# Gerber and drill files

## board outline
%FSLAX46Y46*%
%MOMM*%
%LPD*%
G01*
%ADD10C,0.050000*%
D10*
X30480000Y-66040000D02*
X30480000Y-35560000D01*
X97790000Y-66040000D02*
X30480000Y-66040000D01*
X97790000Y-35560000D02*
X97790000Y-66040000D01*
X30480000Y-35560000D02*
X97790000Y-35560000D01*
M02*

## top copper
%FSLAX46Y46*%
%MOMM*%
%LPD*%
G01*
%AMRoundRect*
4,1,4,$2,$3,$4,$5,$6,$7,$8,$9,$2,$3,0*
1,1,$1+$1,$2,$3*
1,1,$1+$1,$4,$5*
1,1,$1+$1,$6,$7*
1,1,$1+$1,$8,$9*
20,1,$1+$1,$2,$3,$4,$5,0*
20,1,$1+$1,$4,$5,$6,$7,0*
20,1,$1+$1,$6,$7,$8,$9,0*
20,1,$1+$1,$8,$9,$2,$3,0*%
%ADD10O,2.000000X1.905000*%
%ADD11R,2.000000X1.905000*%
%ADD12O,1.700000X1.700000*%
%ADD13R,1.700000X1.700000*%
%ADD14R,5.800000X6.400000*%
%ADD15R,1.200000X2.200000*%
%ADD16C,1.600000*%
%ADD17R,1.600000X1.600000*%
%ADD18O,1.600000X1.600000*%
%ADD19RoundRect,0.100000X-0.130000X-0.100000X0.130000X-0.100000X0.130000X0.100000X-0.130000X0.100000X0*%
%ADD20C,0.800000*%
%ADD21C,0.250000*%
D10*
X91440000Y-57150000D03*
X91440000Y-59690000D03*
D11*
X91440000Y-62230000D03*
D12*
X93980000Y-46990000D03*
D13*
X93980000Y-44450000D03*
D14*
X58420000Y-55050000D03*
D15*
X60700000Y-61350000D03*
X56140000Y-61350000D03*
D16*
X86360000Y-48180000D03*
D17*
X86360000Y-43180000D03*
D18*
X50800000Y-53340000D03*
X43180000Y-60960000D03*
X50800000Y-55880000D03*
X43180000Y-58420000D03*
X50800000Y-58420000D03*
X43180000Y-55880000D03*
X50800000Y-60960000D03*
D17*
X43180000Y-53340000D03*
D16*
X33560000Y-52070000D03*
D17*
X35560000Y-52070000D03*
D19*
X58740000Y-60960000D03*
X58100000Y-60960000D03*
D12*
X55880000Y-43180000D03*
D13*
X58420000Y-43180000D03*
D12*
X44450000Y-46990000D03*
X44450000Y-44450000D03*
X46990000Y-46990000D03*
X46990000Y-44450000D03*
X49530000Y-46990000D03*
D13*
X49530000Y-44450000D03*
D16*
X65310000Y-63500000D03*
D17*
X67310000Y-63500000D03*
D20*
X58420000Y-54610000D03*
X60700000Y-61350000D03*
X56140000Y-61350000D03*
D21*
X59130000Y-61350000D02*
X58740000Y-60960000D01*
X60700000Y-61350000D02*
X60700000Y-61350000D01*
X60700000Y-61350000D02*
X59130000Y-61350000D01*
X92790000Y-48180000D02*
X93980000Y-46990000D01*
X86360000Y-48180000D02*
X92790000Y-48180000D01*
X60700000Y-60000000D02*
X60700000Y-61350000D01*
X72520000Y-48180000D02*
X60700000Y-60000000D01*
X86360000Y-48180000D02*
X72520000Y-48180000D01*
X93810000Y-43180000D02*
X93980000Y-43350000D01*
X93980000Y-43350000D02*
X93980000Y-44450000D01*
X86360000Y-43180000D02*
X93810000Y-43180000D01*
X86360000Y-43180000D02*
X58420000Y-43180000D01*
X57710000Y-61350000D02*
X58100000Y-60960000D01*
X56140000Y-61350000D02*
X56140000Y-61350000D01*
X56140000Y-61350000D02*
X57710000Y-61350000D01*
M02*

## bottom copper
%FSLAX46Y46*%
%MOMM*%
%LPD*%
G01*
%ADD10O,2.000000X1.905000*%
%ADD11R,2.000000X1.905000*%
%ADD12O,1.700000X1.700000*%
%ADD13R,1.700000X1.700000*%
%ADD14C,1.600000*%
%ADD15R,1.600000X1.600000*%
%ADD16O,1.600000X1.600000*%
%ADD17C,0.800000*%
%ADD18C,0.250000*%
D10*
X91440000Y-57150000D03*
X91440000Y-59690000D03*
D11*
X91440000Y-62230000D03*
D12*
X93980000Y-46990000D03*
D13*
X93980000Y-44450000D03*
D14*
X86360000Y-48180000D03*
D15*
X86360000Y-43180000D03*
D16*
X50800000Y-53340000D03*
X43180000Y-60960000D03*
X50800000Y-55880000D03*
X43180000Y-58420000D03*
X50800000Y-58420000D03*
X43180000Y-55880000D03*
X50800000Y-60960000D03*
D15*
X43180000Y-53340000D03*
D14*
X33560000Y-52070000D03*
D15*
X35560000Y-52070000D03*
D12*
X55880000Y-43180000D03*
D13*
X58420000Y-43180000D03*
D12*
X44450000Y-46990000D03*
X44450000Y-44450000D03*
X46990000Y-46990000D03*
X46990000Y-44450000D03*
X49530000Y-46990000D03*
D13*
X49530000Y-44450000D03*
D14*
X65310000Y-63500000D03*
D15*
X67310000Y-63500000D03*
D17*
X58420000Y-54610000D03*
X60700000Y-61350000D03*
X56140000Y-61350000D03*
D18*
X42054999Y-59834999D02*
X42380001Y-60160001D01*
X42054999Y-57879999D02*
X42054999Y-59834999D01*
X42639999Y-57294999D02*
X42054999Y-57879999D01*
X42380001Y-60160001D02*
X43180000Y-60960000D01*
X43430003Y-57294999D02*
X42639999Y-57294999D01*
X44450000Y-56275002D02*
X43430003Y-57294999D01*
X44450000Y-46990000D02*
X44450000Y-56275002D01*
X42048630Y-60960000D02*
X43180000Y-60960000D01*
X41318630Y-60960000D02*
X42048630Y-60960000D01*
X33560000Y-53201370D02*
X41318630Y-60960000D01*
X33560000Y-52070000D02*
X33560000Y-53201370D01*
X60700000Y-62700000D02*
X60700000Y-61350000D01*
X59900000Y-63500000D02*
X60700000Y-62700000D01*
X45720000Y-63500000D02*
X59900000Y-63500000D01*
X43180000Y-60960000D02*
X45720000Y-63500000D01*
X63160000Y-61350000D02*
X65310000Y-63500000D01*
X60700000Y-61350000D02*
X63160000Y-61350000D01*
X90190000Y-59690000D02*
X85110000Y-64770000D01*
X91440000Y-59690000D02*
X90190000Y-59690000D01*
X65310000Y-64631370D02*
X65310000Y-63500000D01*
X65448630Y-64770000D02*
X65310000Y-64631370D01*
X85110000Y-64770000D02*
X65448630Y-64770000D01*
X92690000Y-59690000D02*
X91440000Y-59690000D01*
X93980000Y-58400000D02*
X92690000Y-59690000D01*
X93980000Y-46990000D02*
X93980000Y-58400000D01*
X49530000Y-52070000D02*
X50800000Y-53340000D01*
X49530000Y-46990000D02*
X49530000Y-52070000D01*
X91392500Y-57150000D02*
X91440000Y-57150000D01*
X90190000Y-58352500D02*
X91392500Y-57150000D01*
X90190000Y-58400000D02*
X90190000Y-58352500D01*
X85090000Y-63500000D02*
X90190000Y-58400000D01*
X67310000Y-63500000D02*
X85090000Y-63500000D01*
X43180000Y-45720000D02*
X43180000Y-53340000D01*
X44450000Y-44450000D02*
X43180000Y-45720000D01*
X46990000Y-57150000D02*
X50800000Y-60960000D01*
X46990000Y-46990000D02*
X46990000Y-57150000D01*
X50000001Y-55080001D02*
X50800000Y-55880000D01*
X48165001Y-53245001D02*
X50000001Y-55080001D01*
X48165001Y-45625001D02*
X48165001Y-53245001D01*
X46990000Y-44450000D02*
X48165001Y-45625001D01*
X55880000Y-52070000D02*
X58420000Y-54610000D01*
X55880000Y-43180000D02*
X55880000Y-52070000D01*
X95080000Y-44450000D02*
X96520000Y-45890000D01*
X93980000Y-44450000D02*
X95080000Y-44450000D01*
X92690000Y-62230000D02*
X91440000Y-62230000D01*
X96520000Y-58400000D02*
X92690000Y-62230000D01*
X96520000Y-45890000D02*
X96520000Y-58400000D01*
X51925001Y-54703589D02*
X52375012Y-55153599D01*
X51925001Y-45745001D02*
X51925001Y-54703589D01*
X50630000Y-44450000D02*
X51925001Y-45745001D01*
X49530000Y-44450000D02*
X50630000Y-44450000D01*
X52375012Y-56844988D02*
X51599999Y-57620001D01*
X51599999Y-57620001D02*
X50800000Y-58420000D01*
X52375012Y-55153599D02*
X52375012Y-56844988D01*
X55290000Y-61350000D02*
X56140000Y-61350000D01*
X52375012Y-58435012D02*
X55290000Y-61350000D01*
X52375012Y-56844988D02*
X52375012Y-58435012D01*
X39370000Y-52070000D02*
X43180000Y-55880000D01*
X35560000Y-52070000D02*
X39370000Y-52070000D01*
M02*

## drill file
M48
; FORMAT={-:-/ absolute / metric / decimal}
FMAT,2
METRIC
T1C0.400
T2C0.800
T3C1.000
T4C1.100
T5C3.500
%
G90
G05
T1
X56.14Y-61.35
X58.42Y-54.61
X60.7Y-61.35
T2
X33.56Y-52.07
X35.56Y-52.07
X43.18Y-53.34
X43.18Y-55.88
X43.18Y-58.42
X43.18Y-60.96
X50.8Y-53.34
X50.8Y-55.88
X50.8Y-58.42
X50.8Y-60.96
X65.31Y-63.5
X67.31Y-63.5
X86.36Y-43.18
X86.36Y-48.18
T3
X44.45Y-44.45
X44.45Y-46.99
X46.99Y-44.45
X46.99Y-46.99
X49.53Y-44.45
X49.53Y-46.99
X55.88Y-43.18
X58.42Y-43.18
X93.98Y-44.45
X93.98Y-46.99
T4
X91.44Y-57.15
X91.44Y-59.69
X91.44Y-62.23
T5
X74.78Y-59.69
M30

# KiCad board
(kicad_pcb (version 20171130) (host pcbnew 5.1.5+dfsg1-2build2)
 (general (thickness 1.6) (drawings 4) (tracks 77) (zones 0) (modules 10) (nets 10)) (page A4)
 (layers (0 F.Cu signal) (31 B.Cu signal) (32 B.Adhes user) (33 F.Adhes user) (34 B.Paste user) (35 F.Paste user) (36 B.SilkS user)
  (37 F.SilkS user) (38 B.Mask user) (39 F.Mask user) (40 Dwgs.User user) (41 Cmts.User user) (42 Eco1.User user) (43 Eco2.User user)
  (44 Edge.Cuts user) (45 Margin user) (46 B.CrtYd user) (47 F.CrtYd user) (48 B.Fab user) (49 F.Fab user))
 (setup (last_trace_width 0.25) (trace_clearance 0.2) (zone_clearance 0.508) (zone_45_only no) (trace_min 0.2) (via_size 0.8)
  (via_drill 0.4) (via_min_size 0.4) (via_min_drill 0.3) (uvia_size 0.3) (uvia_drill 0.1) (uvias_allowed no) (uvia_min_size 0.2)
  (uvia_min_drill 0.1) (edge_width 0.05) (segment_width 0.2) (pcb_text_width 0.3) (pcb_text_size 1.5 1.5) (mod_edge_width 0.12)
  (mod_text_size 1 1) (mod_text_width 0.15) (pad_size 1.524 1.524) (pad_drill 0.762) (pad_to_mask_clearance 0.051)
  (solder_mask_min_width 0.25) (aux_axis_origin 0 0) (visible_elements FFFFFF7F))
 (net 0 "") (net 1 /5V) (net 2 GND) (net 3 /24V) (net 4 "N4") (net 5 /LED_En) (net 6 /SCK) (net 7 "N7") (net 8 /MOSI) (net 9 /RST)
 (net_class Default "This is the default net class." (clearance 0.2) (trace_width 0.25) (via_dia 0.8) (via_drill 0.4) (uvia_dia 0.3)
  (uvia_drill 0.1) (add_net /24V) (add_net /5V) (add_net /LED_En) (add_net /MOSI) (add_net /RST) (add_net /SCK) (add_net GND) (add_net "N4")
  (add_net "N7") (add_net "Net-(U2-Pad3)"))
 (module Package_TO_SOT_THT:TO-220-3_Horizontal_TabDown (layer F.Cu) (at 91.44 62.23 90)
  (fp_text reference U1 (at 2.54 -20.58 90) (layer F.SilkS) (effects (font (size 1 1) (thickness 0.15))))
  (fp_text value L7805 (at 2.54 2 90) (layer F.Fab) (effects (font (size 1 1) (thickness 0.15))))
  (pad 3 thru_hole oval (at 5.08 0 90) (size 1.905 2) (drill 1.1) (layers *.Cu *.Mask) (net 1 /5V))
  (pad 2 thru_hole oval (at 2.54 0 90) (size 1.905 2) (drill 1.1) (layers *.Cu *.Mask) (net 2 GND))
  (pad 1 thru_hole rect (at 0 0 90) (size 1.905 2) (drill 1.1) (layers *.Cu *.Mask) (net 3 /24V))
  (pad "" np_thru_hole oval (at 2.54 -16.66 90) (size 3.5 3.5) (drill 3.5) (layers *.Cu *.Mask)))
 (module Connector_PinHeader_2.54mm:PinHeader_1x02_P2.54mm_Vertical (layer F.Cu) (at 93.98 44.45)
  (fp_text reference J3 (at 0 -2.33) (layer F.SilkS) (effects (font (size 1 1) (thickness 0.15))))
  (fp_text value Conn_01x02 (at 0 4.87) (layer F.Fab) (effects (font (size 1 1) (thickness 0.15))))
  (pad 2 thru_hole oval (at 0 2.54) (size 1.7 1.7) (drill 1) (layers *.Cu *.Mask) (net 2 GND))
  (pad 1 thru_hole rect (at 0 0) (size 1.7 1.7) (drill 1) (layers *.Cu *.Mask) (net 3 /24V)))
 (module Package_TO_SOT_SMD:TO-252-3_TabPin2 (layer F.Cu) (at 58.42 57.15 90)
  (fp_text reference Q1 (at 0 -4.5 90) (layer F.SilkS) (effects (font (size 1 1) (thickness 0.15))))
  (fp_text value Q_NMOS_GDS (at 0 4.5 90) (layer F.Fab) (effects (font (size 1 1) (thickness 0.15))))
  (pad "" smd rect (at 0.425 1.525 90) (size 3.05 2.75) (layers F.Paste))
  (pad "" smd rect (at 3.775 -1.525 90) (size 3.05 2.75) (layers F.Paste))
  (pad "" smd rect (at 0.425 -1.525 90) (size 3.05 2.75) (layers F.Paste))
  (pad "" smd rect (at 3.775 1.525 90) (size 3.05 2.75) (layers F.Paste))
  (pad 2 smd rect (at 2.1 0 90) (size 6.4 5.8) (layers F.Cu F.Mask) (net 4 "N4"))
  (pad 3 smd rect (at -4.2 2.28 90) (size 2.2 1.2) (layers F.Cu F.Paste F.Mask) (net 2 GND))
  (pad 1 smd rect (at -4.2 -2.28 90) (size 2.2 1.2) (layers F.Cu F.Paste F.Mask) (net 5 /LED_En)))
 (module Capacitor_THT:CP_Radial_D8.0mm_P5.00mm (layer F.Cu) (at 86.36 43.18 270)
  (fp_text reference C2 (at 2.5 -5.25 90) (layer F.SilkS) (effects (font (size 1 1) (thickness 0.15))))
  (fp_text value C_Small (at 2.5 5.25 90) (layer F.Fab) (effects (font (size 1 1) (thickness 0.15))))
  (pad 2 thru_hole circle (at 5 0 270) (size 1.6 1.6) (drill 0.8) (layers *.Cu *.Mask) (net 2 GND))
  (pad 1 thru_hole rect (at 0 0 270) (size 1.6 1.6) (drill 0.8) (layers *.Cu *.Mask) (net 3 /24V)))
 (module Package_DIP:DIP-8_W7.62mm (layer F.Cu) (at 43.18 53.34)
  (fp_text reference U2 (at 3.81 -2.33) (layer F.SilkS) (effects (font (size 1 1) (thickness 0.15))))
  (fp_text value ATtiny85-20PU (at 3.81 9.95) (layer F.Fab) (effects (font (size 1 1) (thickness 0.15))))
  (pad 8 thru_hole oval (at 7.62 0) (size 1.6 1.6) (drill 0.8) (layers *.Cu *.Mask) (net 1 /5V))
  (pad 4 thru_hole oval (at 0 7.62) (size 1.6 1.6) (drill 0.8) (layers *.Cu *.Mask) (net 2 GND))
  (pad 7 thru_hole oval (at 7.62 2.54) (size 1.6 1.6) (drill 0.8) (layers *.Cu *.Mask) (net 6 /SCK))
  (pad 3 thru_hole oval (at 0 5.08) (size 1.6 1.6) (drill 0.8) (layers *.Cu *.Mask))
  (pad 6 thru_hole oval (at 7.62 5.08) (size 1.6 1.6) (drill 0.8) (layers *.Cu *.Mask) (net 5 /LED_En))
  (pad 2 thru_hole oval (at 0 2.54) (size 1.6 1.6) (drill 0.8) (layers *.Cu *.Mask) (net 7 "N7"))
  (pad 5 thru_hole oval (at 7.62 7.62) (size 1.6 1.6) (drill 0.8) (layers *.Cu *.Mask) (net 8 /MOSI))
  (pad 1 thru_hole rect (at 0 0) (size 1.6 1.6) (drill 0.8) (layers *.Cu *.Mask) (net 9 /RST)))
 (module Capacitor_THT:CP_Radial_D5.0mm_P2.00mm (layer F.Cu) (at 35.56 52.07 180)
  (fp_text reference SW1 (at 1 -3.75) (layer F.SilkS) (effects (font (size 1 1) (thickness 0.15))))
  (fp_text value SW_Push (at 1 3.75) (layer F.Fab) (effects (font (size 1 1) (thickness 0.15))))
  (pad 2 thru_hole circle (at 2 0 180) (size 1.6 1.6) (drill 0.8) (layers *.Cu *.Mask) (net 2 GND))
  (pad 1 thru_hole rect (at 0 0 180) (size 1.6 1.6) (drill 0.8) (layers *.Cu *.Mask) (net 7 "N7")))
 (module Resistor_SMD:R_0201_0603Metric (layer F.Cu) (at 58.42 60.96)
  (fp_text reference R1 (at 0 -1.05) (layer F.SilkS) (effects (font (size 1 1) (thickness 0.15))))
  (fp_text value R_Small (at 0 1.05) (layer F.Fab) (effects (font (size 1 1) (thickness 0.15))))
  (pad 2 smd roundrect (at 0.32 0) (size 0.46 0.4) (layers F.Cu F.Mask) (roundrect_rratio 0.25) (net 2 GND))
  (pad 1 smd roundrect (at -0.32 0) (size 0.46 0.4) (layers F.Cu F.Mask) (roundrect_rratio 0.25) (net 5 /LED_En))
  (pad "" smd roundrect (at 0.345 0) (size 0.318 0.36) (layers F.Paste) (roundrect_rratio 0.25))
  (pad "" smd roundrect (at -0.345 0) (size 0.318 0.36) (layers F.Paste) (roundrect_rratio 0.25)))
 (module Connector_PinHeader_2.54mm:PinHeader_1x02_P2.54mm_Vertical (layer F.Cu) (at 58.42 43.18 270)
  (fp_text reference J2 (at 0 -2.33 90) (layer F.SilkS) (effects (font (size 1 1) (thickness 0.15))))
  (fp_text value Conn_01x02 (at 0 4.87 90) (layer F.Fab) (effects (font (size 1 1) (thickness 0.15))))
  (pad 2 thru_hole oval (at 0 2.54 270) (size 1.7 1.7) (drill 1) (layers *.Cu *.Mask) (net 4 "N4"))
  (pad 1 thru_hole rect (at 0 0 270) (size 1.7 1.7) (drill 1) (layers *.Cu *.Mask) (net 3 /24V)))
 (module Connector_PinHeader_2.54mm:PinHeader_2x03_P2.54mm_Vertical (layer F.Cu) (at 49.53 44.45 270)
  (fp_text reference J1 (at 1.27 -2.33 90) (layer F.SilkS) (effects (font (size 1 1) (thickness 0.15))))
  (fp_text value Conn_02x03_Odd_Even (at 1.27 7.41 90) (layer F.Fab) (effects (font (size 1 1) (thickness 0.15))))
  (pad 6 thru_hole oval (at 2.54 5.08 270) (size 1.7 1.7) (drill 1) (layers *.Cu *.Mask) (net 2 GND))
  (pad 5 thru_hole oval (at 0 5.08 270) (size 1.7 1.7) (drill 1) (layers *.Cu *.Mask) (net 9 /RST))
  (pad 4 thru_hole oval (at 2.54 2.54 270) (size 1.7 1.7) (drill 1) (layers *.Cu *.Mask) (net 8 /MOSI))
  (pad 3 thru_hole oval (at 0 2.54 270) (size 1.7 1.7) (drill 1) (layers *.Cu *.Mask) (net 6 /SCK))
  (pad 2 thru_hole oval (at 2.54 0 270) (size 1.7 1.7) (drill 1) (layers *.Cu *.Mask) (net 1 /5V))
  (pad 1 thru_hole rect (at 0 0 270) (size 1.7 1.7) (drill 1) (layers *.Cu *.Mask) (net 5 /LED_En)))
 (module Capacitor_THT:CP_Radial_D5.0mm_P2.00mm (layer F.Cu) (at 67.31 63.5 180)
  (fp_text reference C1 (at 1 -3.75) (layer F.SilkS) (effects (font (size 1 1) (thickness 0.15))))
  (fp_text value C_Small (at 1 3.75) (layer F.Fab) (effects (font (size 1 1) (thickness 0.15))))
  (pad 2 thru_hole circle (at 2 0 180) (size 1.6 1.6) (drill 0.8) (layers *.Cu *.Mask) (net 2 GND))
  (pad 1 thru_hole rect (at 0 0 180) (size 1.6 1.6) (drill 0.8) (layers *.Cu *.Mask) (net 1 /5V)))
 (gr_line (start 30.48 66.04) (end 30.48 35.56) (layer Edge.Cuts) (width 0.05))
 (gr_line (start 97.79 66.04) (end 30.48 66.04) (layer Edge.Cuts) (width 0.05))
 (gr_line (start 97.79 35.56) (end 97.79 66.04) (layer Edge.Cuts) (width 0.05))
 (gr_line (start 30.48 35.56) (end 97.79 35.56) (layer Edge.Cuts) (width 0.05))
 (via (at 58.42 54.61) (size 0.8) (drill 0.4) (layers F.Cu B.Cu) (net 4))
 (segment (start 42.054999 59.834999) (end 42.380001 60.160001) (width 0.25) (layer B.Cu) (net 2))
 (segment (start 42.054999 57.879999) (end 42.054999 59.834999) (width 0.25) (layer B.Cu) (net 2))
 (segment (start 42.639999 57.294999) (end 42.054999 57.879999) (width 0.25) (layer B.Cu) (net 2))
 (segment (start 42.380001 60.160001) (end 43.18 60.96) (width 0.25) (layer B.Cu) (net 2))
 (segment (start 43.430003 57.294999) (end 42.639999 57.294999) (width 0.25) (layer B.Cu) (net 2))
 (segment (start 44.45 56.275002) (end 43.430003 57.294999) (width 0.25) (layer B.Cu) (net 2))
 (segment (start 44.45 46.99) (end 44.45 56.275002) (width 0.25) (layer B.Cu) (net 2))
 (segment (start 42.04863 60.96) (end 43.18 60.96) (width 0.25) (layer B.Cu) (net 2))
 (segment (start 41.31863 60.96) (end 42.04863 60.96) (width 0.25) (layer B.Cu) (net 2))
 (segment (start 33.56 53.20137) (end 41.31863 60.96) (width 0.25) (layer B.Cu) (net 2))
 (segment (start 33.56 52.07) (end 33.56 53.20137) (width 0.25) (layer B.Cu) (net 2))
 (segment (start 59.13 61.35) (end 58.74 60.96) (width 0.25) (layer F.Cu) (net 2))
 (segment (start 60.7 61.35) (end 60.7 61.35) (width 0.25) (layer F.Cu) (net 2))
 (segment (start 60.7 61.35) (end 59.13 61.35) (width 0.25) (layer F.Cu) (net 2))
 (via (at 60.7 61.35) (size 0.8) (drill 0.4) (layers F.Cu B.Cu) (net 2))
 (segment (start 60.7 62.7) (end 60.7 61.35) (width 0.25) (layer B.Cu) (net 2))
 (segment (start 59.9 63.5) (end 60.7 62.7) (width 0.25) (layer B.Cu) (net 2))
 (segment (start 45.72 63.5) (end 59.9 63.5) (width 0.25) (layer B.Cu) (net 2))
 (segment (start 43.18 60.96) (end 45.72 63.5) (width 0.25) (layer B.Cu) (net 2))
 (segment (start 63.16 61.35) (end 65.31 63.5) (width 0.25) (layer B.Cu) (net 2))
 (segment (start 60.7 61.35) (end 63.16 61.35) (width 0.25) (layer B.Cu) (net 2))
 (segment (start 92.79 48.18) (end 93.98 46.99) (width 0.25) (layer F.Cu) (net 2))
 (segment (start 86.36 48.18) (end 92.79 48.18) (width 0.25) (layer F.Cu) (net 2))
 (segment (start 60.7 60) (end 60.7 61.35) (width 0.25) (layer F.Cu) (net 2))
 (segment (start 72.52 48.18) (end 60.7 60) (width 0.25) (layer F.Cu) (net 2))
 (segment (start 86.36 48.18) (end 72.52 48.18) (width 0.25) (layer F.Cu) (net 2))
 (segment (start 90.19 59.69) (end 85.11 64.77) (width 0.25) (layer B.Cu) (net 2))
 (segment (start 91.44 59.69) (end 90.19 59.69) (width 0.25) (layer B.Cu) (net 2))
 (segment (start 65.31 64.63137) (end 65.31 63.5) (width 0.25) (layer B.Cu) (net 2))
 (segment (start 65.44863 64.77) (end 65.31 64.63137) (width 0.25) (layer B.Cu) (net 2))
 (segment (start 85.11 64.77) (end 65.44863 64.77) (width 0.25) (layer B.Cu) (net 2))
 (segment (start 92.69 59.69) (end 91.44 59.69) (width 0.25) (layer B.Cu) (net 2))
 (segment (start 93.98 58.4) (end 92.69 59.69) (width 0.25) (layer B.Cu) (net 2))
 (segment (start 93.98 46.99) (end 93.98 58.4) (width 0.25) (layer B.Cu) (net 2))
 (segment (start 49.53 52.07) (end 50.8 53.34) (width 0.25) (layer B.Cu) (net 1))
 (segment (start 49.53 46.99) (end 49.53 52.07) (width 0.25) (layer B.Cu) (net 1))
 (segment (start 91.3925 57.15) (end 91.44 57.15) (width 0.25) (layer B.Cu) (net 1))
 (segment (start 90.19 58.3525) (end 91.3925 57.15) (width 0.25) (layer B.Cu) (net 1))
 (segment (start 90.19 58.4) (end 90.19 58.3525) (width 0.25) (layer B.Cu) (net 1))
 (segment (start 85.09 63.5) (end 90.19 58.4) (width 0.25) (layer B.Cu) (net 1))
 (segment (start 67.31 63.5) (end 85.09 63.5) (width 0.25) (layer B.Cu) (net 1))
 (segment (start 43.18 45.72) (end 43.18 53.34) (width 0.25) (layer B.Cu) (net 9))
 (segment (start 44.45 44.45) (end 43.18 45.72) (width 0.25) (layer B.Cu) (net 9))
 (segment (start 46.99 57.15) (end 50.8 60.96) (width 0.25) (layer B.Cu) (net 8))
 (segment (start 46.99 46.99) (end 46.99 57.15) (width 0.25) (layer B.Cu) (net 8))
 (segment (start 50.000001 55.080001) (end 50.8 55.88) (width 0.25) (layer B.Cu) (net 6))
 (segment (start 48.165001 53.245001) (end 50.000001 55.080001) (width 0.25) (layer B.Cu) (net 6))
 (segment (start 48.165001 45.625001) (end 48.165001 53.245001) (width 0.25) (layer B.Cu) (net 6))
 (segment (start 46.99 44.45) (end 48.165001 45.625001) (width 0.25) (layer B.Cu) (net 6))
 (segment (start 55.88 52.07) (end 58.42 54.61) (width 0.25) (layer B.Cu) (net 4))
 (segment (start 55.88 43.18) (end 55.88 52.07) (width 0.25) (layer B.Cu) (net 4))
 (segment (start 93.81 43.18) (end 93.98 43.35) (width 0.25) (layer F.Cu) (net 3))
 (segment (start 93.98 43.35) (end 93.98 44.45) (width 0.25) (layer F.Cu) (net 3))
 (segment (start 86.36 43.18) (end 93.81 43.18) (width 0.25) (layer F.Cu) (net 3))
 (segment (start 86.36 43.18) (end 58.42 43.18) (width 0.25) (layer F.Cu) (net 3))
 (segment (start 95.08 44.45) (end 96.52 45.89) (width 0.25) (layer B.Cu) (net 3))
 (segment (start 93.98 44.45) (end 95.08 44.45) (width 0.25) (layer B.Cu) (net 3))
 (segment (start 92.69 62.23) (end 91.44 62.23) (width 0.25) (layer B.Cu) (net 3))
 (segment (start 96.52 58.4) (end 92.69 62.23) (width 0.25) (layer B.Cu) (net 3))
 (segment (start 96.52 45.89) (end 96.52 58.4) (width 0.25) (layer B.Cu) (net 3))
 (segment (start 51.925001 54.703589) (end 52.375012 55.153599) (width 0.25) (layer B.Cu) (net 5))
 (segment (start 51.925001 45.745001) (end 51.925001 54.703589) (width 0.25) (layer B.Cu) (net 5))
 (segment (start 50.63 44.45) (end 51.925001 45.745001) (width 0.25) (layer B.Cu) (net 5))
 (segment (start 49.53 44.45) (end 50.63 44.45) (width 0.25) (layer B.Cu) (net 5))
 (segment (start 52.375012 56.844988) (end 51.599999 57.620001) (width 0.25) (layer B.Cu) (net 5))
 (segment (start 51.599999 57.620001) (end 50.8 58.42) (width 0.25) (layer B.Cu) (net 5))
 (segment (start 52.375012 55.153599) (end 52.375012 56.844988) (width 0.25) (layer B.Cu) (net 5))
 (segment (start 57.71 61.35) (end 58.1 60.96) (width 0.25) (layer F.Cu) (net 5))
 (segment (start 56.14 61.35) (end 56.14 61.35) (width 0.25) (layer F.Cu) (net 5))
 (segment (start 56.14 61.35) (end 57.71 61.35) (width 0.25) (layer F.Cu) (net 5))
 (via (at 56.14 61.35) (size 0.8) (drill 0.4) (layers F.Cu B.Cu) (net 5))
 (segment (start 55.29 61.35) (end 56.14 61.35) (width 0.25) (layer B.Cu) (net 5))
 (segment (start 52.375012 58.435012) (end 55.29 61.35) (width 0.25) (layer B.Cu) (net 5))
 (segment (start 52.375012 56.844988) (end 52.375012 58.435012) (width 0.25) (layer B.Cu) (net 5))
 (segment (start 39.37 52.07) (end 43.18 55.88) (width 0.25) (layer B.Cu) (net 7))
 (segment (start 35.56 52.07) (end 39.37 52.07) (width 0.25) (layer B.Cu) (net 7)))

